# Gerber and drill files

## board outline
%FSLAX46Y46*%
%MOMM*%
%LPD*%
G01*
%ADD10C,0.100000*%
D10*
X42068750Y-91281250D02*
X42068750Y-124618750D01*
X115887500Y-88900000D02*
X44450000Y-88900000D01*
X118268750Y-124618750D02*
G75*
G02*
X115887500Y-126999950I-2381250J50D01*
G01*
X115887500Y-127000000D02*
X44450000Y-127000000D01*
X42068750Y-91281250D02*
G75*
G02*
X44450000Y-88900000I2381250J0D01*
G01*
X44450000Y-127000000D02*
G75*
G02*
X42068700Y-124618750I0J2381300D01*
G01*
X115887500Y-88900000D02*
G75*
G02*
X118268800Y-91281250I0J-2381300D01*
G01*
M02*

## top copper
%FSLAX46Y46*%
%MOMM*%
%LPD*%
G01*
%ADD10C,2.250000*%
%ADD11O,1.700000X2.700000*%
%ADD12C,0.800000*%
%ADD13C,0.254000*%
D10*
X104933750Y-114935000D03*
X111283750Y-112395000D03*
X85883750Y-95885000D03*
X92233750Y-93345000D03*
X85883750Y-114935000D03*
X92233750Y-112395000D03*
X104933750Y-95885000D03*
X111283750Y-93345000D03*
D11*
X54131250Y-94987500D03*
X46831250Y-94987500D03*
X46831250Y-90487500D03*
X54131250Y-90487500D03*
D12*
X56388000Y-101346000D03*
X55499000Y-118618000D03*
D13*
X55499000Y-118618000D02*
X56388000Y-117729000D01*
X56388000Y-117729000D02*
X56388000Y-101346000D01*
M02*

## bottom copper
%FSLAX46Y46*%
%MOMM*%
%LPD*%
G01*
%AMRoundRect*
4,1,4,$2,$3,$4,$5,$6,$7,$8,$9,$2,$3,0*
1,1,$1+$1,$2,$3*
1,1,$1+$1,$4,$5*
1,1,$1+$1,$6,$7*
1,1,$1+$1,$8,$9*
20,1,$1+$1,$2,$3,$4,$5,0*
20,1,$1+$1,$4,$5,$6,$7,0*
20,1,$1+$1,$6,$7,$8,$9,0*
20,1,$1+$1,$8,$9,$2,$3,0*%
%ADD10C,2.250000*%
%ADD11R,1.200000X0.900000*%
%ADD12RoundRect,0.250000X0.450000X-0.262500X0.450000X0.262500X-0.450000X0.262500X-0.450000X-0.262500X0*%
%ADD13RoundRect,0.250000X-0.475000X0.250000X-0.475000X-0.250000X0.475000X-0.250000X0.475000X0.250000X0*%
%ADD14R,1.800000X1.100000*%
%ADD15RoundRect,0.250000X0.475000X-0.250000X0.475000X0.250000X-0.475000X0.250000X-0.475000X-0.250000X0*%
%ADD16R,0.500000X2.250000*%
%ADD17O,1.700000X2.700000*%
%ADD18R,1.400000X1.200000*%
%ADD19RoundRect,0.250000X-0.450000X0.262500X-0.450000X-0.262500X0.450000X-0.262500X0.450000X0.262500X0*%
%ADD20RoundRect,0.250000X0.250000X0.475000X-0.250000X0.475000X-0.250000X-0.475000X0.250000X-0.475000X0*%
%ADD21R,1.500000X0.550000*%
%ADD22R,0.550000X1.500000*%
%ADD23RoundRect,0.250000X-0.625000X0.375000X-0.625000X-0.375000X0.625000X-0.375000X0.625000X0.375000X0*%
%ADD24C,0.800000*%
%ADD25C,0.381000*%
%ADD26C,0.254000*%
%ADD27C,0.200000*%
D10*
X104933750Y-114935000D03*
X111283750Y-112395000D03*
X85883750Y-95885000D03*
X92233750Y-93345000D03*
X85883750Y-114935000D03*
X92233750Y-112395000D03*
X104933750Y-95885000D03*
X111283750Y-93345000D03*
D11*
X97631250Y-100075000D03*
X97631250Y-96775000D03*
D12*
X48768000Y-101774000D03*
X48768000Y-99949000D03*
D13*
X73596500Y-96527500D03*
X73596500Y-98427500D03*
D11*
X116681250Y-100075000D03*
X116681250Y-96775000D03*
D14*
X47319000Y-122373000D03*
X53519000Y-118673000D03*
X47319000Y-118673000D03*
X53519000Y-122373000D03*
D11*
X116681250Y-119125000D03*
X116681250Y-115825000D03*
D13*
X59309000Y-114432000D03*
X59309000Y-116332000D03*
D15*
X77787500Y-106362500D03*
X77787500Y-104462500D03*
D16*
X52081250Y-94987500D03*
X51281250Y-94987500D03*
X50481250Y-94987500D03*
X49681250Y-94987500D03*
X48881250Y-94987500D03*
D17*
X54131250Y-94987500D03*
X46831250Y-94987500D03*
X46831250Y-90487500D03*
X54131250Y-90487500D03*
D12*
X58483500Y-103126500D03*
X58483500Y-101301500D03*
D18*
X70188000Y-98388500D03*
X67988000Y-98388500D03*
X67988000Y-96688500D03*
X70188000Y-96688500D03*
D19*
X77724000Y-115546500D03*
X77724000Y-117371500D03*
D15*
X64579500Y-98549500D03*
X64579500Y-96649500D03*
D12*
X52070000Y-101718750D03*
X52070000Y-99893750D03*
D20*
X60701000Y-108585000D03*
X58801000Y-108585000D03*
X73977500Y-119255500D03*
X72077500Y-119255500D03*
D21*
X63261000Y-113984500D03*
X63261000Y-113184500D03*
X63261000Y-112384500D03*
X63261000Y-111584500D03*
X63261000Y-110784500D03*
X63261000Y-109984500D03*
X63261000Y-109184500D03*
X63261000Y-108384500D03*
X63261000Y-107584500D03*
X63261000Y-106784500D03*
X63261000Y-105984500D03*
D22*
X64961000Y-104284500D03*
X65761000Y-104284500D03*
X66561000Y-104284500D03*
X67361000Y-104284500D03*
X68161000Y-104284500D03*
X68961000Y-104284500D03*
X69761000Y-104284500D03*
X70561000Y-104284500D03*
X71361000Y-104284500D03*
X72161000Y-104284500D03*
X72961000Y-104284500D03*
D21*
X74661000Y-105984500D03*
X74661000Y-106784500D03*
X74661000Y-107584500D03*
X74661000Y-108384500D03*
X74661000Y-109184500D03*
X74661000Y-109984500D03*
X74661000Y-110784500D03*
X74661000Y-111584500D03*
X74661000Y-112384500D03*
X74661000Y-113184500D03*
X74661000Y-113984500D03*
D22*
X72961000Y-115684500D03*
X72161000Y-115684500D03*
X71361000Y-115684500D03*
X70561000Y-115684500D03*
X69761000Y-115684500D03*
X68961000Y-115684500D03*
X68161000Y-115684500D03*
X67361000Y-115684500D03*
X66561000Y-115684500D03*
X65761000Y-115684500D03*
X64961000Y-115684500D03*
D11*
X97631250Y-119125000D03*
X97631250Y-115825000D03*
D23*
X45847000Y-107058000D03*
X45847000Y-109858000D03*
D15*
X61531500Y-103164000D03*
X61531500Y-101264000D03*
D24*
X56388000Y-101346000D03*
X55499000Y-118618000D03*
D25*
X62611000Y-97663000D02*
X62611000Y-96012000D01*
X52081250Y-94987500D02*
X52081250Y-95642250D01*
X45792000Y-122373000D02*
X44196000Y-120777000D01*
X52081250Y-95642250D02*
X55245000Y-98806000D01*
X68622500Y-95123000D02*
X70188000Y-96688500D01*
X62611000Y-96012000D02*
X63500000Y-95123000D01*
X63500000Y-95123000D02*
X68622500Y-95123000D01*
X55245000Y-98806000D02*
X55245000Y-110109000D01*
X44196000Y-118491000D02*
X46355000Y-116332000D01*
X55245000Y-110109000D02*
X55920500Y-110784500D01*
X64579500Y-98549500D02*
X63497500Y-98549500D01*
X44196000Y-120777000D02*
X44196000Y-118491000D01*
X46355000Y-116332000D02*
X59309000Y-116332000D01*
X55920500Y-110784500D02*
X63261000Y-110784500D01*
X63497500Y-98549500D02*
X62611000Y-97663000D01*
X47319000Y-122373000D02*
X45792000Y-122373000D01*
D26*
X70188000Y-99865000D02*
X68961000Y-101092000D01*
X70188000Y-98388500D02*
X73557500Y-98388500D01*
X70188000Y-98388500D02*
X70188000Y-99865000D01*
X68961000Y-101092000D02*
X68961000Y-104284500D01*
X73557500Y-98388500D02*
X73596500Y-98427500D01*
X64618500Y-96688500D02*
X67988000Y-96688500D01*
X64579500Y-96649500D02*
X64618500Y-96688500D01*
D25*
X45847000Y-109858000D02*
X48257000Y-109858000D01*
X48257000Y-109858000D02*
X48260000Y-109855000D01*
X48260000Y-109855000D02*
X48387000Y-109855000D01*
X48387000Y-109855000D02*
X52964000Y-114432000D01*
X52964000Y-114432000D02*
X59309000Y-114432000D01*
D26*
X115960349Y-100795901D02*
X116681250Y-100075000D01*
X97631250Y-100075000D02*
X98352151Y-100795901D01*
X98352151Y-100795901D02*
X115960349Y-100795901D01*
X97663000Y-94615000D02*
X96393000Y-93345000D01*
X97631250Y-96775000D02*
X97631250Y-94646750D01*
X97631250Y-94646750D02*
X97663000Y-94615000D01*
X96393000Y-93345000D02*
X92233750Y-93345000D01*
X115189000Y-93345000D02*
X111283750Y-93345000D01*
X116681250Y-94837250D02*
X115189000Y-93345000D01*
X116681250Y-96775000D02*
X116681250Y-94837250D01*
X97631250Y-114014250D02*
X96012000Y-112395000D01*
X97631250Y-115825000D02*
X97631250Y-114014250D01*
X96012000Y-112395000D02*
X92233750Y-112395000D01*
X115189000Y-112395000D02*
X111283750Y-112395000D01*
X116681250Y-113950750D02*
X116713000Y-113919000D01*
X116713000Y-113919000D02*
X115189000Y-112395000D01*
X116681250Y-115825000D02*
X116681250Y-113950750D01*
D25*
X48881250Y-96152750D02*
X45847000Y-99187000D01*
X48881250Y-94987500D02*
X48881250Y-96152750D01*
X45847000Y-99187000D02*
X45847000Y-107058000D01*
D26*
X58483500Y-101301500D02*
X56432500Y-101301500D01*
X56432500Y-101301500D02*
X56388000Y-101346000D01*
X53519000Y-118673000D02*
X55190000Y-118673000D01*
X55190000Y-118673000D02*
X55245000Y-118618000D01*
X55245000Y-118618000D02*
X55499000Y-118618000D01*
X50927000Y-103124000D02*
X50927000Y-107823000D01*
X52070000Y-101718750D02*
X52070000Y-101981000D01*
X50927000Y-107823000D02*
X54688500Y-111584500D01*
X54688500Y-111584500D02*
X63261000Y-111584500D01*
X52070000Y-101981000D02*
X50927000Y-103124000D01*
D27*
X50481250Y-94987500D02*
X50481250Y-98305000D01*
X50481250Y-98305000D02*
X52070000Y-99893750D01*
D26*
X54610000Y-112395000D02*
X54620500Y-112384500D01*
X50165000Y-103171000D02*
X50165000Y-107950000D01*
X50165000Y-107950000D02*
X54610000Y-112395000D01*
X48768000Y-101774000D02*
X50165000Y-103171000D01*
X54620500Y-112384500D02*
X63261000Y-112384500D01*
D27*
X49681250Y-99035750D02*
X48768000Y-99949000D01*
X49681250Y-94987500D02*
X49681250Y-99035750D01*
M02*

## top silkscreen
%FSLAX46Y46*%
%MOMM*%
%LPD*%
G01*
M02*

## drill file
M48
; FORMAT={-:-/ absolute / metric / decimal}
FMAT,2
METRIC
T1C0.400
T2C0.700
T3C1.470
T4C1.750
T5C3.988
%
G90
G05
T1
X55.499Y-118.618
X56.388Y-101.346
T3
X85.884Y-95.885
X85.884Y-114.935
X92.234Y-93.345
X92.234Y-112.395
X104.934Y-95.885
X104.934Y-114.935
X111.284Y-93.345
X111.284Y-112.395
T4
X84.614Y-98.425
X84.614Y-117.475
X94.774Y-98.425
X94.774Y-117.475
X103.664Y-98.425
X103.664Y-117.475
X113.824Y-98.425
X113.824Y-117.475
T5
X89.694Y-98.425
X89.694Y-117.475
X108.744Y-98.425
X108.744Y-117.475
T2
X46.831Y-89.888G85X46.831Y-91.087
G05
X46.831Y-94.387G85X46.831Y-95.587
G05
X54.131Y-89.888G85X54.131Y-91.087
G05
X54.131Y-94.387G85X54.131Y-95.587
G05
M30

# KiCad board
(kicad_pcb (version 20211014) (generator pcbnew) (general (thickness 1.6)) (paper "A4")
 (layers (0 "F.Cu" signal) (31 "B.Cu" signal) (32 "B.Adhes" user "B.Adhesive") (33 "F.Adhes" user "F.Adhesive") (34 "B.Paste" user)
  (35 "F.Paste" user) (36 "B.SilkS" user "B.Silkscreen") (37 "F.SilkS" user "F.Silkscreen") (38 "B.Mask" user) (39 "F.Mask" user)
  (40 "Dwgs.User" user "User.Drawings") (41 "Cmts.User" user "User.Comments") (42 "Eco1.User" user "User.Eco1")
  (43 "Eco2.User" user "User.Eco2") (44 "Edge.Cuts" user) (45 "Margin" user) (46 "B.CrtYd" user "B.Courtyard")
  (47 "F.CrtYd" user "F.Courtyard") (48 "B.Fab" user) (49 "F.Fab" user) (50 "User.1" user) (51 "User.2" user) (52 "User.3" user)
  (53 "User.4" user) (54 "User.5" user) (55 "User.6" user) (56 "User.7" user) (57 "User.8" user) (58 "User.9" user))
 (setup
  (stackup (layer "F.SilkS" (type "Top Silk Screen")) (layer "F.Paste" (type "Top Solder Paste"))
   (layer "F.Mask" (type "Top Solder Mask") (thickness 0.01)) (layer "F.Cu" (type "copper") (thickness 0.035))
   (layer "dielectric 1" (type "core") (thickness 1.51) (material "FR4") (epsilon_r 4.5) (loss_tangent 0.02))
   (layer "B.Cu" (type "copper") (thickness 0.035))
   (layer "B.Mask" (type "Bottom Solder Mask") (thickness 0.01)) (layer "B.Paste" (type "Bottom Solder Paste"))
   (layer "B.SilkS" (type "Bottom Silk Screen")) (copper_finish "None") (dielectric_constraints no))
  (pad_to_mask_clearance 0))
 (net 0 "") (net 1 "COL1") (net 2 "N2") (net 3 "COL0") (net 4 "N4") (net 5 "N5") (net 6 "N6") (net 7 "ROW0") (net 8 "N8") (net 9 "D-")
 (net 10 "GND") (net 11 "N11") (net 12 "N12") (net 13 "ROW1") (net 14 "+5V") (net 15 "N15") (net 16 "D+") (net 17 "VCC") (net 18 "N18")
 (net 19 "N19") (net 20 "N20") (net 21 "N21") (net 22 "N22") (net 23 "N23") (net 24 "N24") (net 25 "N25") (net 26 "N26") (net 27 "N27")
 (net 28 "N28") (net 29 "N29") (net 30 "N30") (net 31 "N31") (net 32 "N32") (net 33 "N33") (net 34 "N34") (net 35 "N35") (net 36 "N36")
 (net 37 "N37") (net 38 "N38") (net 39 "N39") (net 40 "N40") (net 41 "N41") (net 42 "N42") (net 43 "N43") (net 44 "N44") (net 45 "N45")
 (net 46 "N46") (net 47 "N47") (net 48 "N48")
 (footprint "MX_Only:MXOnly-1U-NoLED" (layer "F.Cu") (at 108.74375 117.475)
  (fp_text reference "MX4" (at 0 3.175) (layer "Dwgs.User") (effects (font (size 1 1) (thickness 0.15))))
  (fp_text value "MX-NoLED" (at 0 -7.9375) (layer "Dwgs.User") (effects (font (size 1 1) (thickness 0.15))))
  (pad "" np_thru_hole circle locked (at 5.08 0 48.0996) (size 1.75 1.75) (drill 1.75) (layers *.Cu *.Mask))
  (pad "" np_thru_hole circle locked (at 0 0) (size 3.9878 3.9878) (drill 3.9878) (layers *.Cu *.Mask))
  (pad "" np_thru_hole circle locked (at -5.08 0 48.0996) (size 1.75 1.75) (drill 1.75) (layers *.Cu *.Mask))
  (pad "1" thru_hole circle locked (at -3.81 -2.54) (size 2.25 2.25) (drill 1.47) (layers *.Cu "B.Mask") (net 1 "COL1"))
  (pad "2" thru_hole circle locked (at 2.54 -5.08) (size 2.25 2.25) (drill 1.47) (layers *.Cu "B.Mask") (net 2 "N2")))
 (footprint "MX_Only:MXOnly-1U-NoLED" (layer "F.Cu") (at 89.69375 98.425)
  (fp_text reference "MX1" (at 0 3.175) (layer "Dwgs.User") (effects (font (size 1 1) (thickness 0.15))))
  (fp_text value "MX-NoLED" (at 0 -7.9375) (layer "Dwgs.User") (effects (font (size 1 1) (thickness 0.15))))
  (pad "" np_thru_hole circle locked (at -5.08 0 48.0996) (size 1.75 1.75) (drill 1.75) (layers *.Cu *.Mask))
  (pad "" np_thru_hole circle locked (at 5.08 0 48.0996) (size 1.75 1.75) (drill 1.75) (layers *.Cu *.Mask))
  (pad "" np_thru_hole circle locked (at 0 0) (size 3.9878 3.9878) (drill 3.9878) (layers *.Cu *.Mask))
  (pad "1" thru_hole circle locked (at -3.81 -2.54) (size 2.25 2.25) (drill 1.47) (layers *.Cu "B.Mask") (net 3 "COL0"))
  (pad "2" thru_hole circle locked (at 2.54 -5.08) (size 2.25 2.25) (drill 1.47) (layers *.Cu "B.Mask") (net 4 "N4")))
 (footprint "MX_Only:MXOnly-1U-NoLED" (layer "F.Cu") (at 89.69375 117.475)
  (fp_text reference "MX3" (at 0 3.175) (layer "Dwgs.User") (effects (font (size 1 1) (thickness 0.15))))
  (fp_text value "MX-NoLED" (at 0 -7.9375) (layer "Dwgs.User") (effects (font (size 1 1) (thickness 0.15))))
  (pad "" np_thru_hole circle locked (at -5.08 0 48.0996) (size 1.75 1.75) (drill 1.75) (layers *.Cu *.Mask))
  (pad "" np_thru_hole circle locked (at 5.08 0 48.0996) (size 1.75 1.75) (drill 1.75) (layers *.Cu *.Mask))
  (pad "" np_thru_hole circle locked (at 0 0) (size 3.9878 3.9878) (drill 3.9878) (layers *.Cu *.Mask))
  (pad "1" thru_hole circle locked (at -3.81 -2.54) (size 2.25 2.25) (drill 1.47) (layers *.Cu "B.Mask") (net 3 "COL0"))
  (pad "2" thru_hole circle locked (at 2.54 -5.08) (size 2.25 2.25) (drill 1.47) (layers *.Cu "B.Mask") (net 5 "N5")))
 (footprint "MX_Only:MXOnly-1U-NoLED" (layer "F.Cu") (at 108.74375 98.425)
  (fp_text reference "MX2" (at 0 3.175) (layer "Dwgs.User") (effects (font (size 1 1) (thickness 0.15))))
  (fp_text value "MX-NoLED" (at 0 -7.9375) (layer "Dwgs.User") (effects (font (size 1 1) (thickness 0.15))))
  (pad "" np_thru_hole circle locked (at -5.08 0 48.0996) (size 1.75 1.75) (drill 1.75) (layers *.Cu *.Mask))
  (pad "" np_thru_hole circle locked (at 0 0) (size 3.9878 3.9878) (drill 3.9878) (layers *.Cu *.Mask))
  (pad "" np_thru_hole circle locked (at 5.08 0 48.0996) (size 1.75 1.75) (drill 1.75) (layers *.Cu *.Mask))
  (pad "1" thru_hole circle locked (at -3.81 -2.54) (size 2.25 2.25) (drill 1.47) (layers *.Cu "B.Mask") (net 1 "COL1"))
  (pad "2" thru_hole circle locked (at 2.54 -5.08) (size 2.25 2.25) (drill 1.47) (layers *.Cu "B.Mask") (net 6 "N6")))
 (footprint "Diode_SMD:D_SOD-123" (layer "B.Cu") (at 97.63125 98.425 90)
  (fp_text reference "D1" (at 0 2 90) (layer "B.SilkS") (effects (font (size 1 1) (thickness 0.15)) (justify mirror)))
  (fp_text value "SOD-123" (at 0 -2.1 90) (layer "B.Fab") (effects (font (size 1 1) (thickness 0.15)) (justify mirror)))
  (pad "1" smd rect (at -1.65 0 90) (size 0.9 1.2) (layers "B.Cu" "B.Paste" "B.Mask") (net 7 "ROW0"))
  (pad "2" smd rect (at 1.65 0 90) (size 0.9 1.2) (layers "B.Cu" "B.Paste" "B.Mask") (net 4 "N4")))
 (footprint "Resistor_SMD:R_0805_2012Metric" (layer "B.Cu") (at 48.768 100.8615 90)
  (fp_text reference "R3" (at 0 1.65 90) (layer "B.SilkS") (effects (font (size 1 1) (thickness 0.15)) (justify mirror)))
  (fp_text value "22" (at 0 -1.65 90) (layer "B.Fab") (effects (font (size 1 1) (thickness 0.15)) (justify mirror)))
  (pad "1" smd roundrect (at -0.9125 0 90) (size 1.025 1.4) (layers "B.Cu" "B.Paste" "B.Mask") (roundrect_rratio 0.243902) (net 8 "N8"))
  (pad "2" smd roundrect (at 0.9125 0 90) (size 1.025 1.4) (layers "B.Cu" "B.Paste" "B.Mask") (roundrect_rratio 0.243902) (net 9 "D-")))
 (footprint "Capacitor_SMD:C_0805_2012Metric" (layer "B.Cu") (at 73.5965 97.4775 -90)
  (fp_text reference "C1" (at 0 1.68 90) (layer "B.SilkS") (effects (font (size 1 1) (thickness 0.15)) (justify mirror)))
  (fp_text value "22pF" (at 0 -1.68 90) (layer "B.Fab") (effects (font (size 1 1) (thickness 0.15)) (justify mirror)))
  (pad "1" smd roundrect (at -0.95 0 270) (size 1 1.45) (layers "B.Cu" "B.Paste" "B.Mask") (roundrect_rratio 0.25) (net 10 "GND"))
  (pad "2" smd roundrect (at 0.95 0 270) (size 1 1.45) (layers "B.Cu" "B.Paste" "B.Mask") (roundrect_rratio 0.25) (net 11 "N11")))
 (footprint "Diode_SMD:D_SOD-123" (layer "B.Cu") (at 116.68125 98.425 90)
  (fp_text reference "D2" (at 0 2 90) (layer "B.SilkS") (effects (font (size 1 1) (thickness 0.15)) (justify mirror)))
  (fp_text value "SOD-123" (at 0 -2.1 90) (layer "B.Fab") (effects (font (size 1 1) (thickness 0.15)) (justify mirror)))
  (pad "1" smd rect (at -1.65 0 90) (size 0.9 1.2) (layers "B.Cu" "B.Paste" "B.Mask") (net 7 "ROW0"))
  (pad "2" smd rect (at 1.65 0 90) (size 0.9 1.2) (layers "B.Cu" "B.Paste" "B.Mask") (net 6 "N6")))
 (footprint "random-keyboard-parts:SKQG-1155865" (layer "B.Cu") (at 50.419 120.523 180)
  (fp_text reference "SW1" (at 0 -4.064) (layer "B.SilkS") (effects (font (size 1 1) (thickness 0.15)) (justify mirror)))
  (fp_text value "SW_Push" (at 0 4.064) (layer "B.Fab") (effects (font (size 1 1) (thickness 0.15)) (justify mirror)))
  (pad "1" smd rect locked (at 3.1 -1.85 180) (size 1.8 1.1) (layers "B.Cu" "B.Paste" "B.Mask") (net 10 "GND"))
  (pad "2" smd rect locked (at -3.1 1.85 180) (size 1.8 1.1) (layers "B.Cu" "B.Paste" "B.Mask") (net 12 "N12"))
  (pad "3" smd rect locked (at 3.1 1.85 180) (size 1.8 1.1) (layers "B.Cu" "B.Paste" "B.Mask"))
  (pad "4" smd rect locked (at -3.1 -1.85 180) (size 1.8 1.1) (layers "B.Cu" "B.Paste" "B.Mask")))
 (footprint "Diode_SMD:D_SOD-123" (layer "B.Cu") (at 116.68125 117.475 90)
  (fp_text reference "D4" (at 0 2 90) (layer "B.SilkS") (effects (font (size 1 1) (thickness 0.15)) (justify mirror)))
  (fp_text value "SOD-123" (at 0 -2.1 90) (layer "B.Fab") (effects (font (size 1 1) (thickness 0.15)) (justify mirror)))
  (pad "1" smd rect (at -1.65 0 90) (size 0.9 1.2) (layers "B.Cu" "B.Paste" "B.Mask") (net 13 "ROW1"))
  (pad "2" smd rect (at 1.65 0 90) (size 0.9 1.2) (layers "B.Cu" "B.Paste" "B.Mask") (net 2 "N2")))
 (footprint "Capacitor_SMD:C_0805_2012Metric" (layer "B.Cu") (at 59.309 115.382 -90)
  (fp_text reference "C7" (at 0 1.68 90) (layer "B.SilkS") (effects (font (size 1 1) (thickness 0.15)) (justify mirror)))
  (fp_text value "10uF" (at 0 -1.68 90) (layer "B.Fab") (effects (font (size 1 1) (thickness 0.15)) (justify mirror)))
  (pad "1" smd roundrect (at -0.95 0 270) (size 1 1.45) (layers "B.Cu" "B.Paste" "B.Mask") (roundrect_rratio 0.25) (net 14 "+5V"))
  (pad "2" smd roundrect (at 0.95 0 270) (size 1 1.45) (layers "B.Cu" "B.Paste" "B.Mask") (roundrect_rratio 0.25) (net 10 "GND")))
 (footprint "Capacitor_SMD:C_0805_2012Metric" (layer "B.Cu") (at 77.7875 105.4125 90)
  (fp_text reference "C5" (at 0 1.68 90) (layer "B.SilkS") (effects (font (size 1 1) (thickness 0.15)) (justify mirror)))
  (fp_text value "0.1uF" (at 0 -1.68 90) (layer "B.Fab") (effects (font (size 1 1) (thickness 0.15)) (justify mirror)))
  (pad "1" smd roundrect (at -0.95 0 90) (size 1 1.45) (layers "B.Cu" "B.Paste" "B.Mask") (roundrect_rratio 0.25) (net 14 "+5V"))
  (pad "2" smd roundrect (at 0.95 0 90) (size 1 1.45) (layers "B.Cu" "B.Paste" "B.Mask") (roundrect_rratio 0.25) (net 10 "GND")))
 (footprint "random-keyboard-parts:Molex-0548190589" (layer "B.Cu") (at 50.48125 90.4875 -90)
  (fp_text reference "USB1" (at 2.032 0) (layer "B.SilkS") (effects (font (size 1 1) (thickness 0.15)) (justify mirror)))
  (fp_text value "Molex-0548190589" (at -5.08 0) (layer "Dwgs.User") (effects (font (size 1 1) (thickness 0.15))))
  (pad "1" smd rect locked (at 4.5 -1.6 270) (size 2.25 0.5) (layers "B.Cu" "B.Paste" "B.Mask") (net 10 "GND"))
  (pad "2" smd rect locked (at 4.5 -0.8 270) (size 2.25 0.5) (layers "B.Cu" "B.Paste" "B.Mask") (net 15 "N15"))
  (pad "3" smd rect locked (at 4.5 0 270) (size 2.25 0.5) (layers "B.Cu" "B.Paste" "B.Mask") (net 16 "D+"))
  (pad "4" smd rect locked (at 4.5 0.8 270) (size 2.25 0.5) (layers "B.Cu" "B.Paste" "B.Mask") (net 9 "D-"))
  (pad "5" smd rect locked (at 4.5 1.6 270) (size 2.25 0.5) (layers "B.Cu" "B.Paste" "B.Mask") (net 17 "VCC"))
  (pad "6" thru_hole oval locked (at 4.5 -3.65 270) (size 2.7 1.7) (drill oval 1.9 0.7) (layers *.Cu *.Mask) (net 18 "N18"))
  (pad "6" thru_hole oval locked (at 4.5 3.65 270) (size 2.7 1.7) (drill oval 1.9 0.7) (layers *.Cu *.Mask) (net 18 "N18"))
  (pad "6" thru_hole oval locked (at 0 3.65 270) (size 2.7 1.7) (drill oval 1.9 0.7) (layers *.Cu *.Mask) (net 18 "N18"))
  (pad "6" thru_hole oval locked (at 0 -3.65 270) (size 2.7 1.7) (drill oval 1.9 0.7) (layers *.Cu *.Mask) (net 18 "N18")))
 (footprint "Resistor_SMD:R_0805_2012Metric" (layer "B.Cu") (at 58.4835 102.214 90)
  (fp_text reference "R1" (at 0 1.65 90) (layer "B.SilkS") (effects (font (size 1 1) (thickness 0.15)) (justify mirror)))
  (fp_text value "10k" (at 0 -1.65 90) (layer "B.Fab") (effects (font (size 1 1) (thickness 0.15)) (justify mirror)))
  (pad "1" smd roundrect (at -0.9125 0 90) (size 1.025 1.4) (layers "B.Cu" "B.Paste" "B.Mask") (roundrect_rratio 0.243902) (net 14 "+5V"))
  (pad "2" smd roundrect (at 0.9125 0 90) (size 1.025 1.4) (layers "B.Cu" "B.Paste" "B.Mask") (roundrect_rratio 0.243902) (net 12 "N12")))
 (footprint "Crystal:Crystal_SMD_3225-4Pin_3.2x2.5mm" (layer "B.Cu") (at 69.088 97.5385 180)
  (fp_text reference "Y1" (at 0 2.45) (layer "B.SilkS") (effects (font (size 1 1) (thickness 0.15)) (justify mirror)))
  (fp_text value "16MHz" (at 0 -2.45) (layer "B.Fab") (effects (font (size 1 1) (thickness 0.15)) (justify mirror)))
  (pad "1" smd rect (at -1.1 -0.85 180) (size 1.4 1.2) (layers "B.Cu" "B.Paste" "B.Mask") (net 11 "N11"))
  (pad "2" smd rect (at 1.1 -0.85 180) (size 1.4 1.2) (layers "B.Cu" "B.Paste" "B.Mask") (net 10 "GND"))
  (pad "3" smd rect (at 1.1 0.85 180) (size 1.4 1.2) (layers "B.Cu" "B.Paste" "B.Mask") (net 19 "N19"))
  (pad "4" smd rect (at -1.1 0.85 180) (size 1.4 1.2) (layers "B.Cu" "B.Paste" "B.Mask") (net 10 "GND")))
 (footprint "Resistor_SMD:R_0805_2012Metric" (layer "B.Cu") (at 77.724 116.459 -90)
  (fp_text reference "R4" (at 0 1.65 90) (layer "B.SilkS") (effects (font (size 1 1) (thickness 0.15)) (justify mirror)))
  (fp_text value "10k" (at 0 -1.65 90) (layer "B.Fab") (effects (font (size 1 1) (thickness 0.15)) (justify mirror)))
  (pad "1" smd roundrect (at -0.9125 0 270) (size 1.025 1.4) (layers "B.Cu" "B.Paste" "B.Mask") (roundrect_rratio 0.243902) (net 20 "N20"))
  (pad "2" smd roundrect (at 0.9125 0 270) (size 1.025 1.4) (layers "B.Cu" "B.Paste" "B.Mask") (roundrect_rratio 0.243902) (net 10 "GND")))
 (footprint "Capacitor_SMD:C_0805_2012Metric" (layer "B.Cu") (at 64.5795 97.5995 90)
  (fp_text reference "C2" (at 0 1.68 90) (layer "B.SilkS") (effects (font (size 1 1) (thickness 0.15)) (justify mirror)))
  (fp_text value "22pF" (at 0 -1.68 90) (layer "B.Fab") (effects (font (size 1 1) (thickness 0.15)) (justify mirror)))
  (pad "1" smd roundrect (at -0.95 0 90) (size 1 1.45) (layers "B.Cu" "B.Paste" "B.Mask") (roundrect_rratio 0.25) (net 10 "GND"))
  (pad "2" smd roundrect (at 0.95 0 90) (size 1 1.45) (layers "B.Cu" "B.Paste" "B.Mask") (roundrect_rratio 0.25) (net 19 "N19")))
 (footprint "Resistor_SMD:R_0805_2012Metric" (layer "B.Cu") (at 52.07 100.80625 90)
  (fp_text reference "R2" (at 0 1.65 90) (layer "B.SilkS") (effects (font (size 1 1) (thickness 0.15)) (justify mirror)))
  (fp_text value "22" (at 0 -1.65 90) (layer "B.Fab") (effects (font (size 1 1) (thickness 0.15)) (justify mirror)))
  (pad "1" smd roundrect (at -0.9125 0 90) (size 1.025 1.4) (layers "B.Cu" "B.Paste" "B.Mask") (roundrect_rratio 0.243902) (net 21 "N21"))
  (pad "2" smd roundrect (at 0.9125 0 90) (size 1.025 1.4) (layers "B.Cu" "B.Paste" "B.Mask") (roundrect_rratio 0.243902) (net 16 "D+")))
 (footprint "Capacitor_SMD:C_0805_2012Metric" (layer "B.Cu") (at 59.751 108.585 180)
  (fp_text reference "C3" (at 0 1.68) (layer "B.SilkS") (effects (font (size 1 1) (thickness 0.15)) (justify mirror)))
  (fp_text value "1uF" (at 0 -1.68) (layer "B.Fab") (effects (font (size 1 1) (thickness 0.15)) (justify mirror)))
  (pad "1" smd roundrect (at -0.95 0 180) (size 1 1.45) (layers "B.Cu" "B.Paste" "B.Mask") (roundrect_rratio 0.25) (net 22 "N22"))
  (pad "2" smd roundrect (at 0.95 0 180) (size 1 1.45) (layers "B.Cu" "B.Paste" "B.Mask") (roundrect_rratio 0.25) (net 10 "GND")))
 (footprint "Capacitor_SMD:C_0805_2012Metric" (layer "B.Cu") (at 73.0275 119.2555 180)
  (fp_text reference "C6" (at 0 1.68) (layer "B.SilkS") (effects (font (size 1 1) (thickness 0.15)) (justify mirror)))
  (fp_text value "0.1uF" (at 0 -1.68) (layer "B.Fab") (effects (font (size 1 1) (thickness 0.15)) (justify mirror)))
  (pad "1" smd roundrect (at -0.95 0 180) (size 1 1.45) (layers "B.Cu" "B.Paste" "B.Mask") (roundrect_rratio 0.25) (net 14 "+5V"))
  (pad "2" smd roundrect (at 0.95 0 180) (size 1 1.45) (layers "B.Cu" "B.Paste" "B.Mask") (roundrect_rratio 0.25) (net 10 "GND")))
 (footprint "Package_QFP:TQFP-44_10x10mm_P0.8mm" (layer "B.Cu") (at 68.961 109.9845)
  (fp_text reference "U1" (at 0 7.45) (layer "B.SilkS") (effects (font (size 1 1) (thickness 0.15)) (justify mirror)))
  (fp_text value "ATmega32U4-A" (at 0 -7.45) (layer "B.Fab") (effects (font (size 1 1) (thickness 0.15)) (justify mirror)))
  (pad "1" smd rect (at -5.7 4) (size 1.5 0.55) (layers "B.Cu" "B.Paste" "B.Mask") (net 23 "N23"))
  (pad "2" smd rect (at -5.7 3.2) (size 1.5 0.55) (layers "B.Cu" "B.Paste" "B.Mask") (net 14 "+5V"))
  (pad "3" smd rect (at -5.7 2.4) (size 1.5 0.55) (layers "B.Cu" "B.Paste" "B.Mask") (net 8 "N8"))
  (pad "4" smd rect (at -5.7 1.6) (size 1.5 0.55) (layers "B.Cu" "B.Paste" "B.Mask") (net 21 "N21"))
  (pad "5" smd rect (at -5.7 0.8) (size 1.5 0.55) (layers "B.Cu" "B.Paste" "B.Mask") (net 10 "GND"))
  (pad "6" smd rect (at -5.7 0) (size 1.5 0.55) (layers "B.Cu" "B.Paste" "B.Mask") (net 22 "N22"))
  (pad "7" smd rect (at -5.7 -0.8) (size 1.5 0.55) (layers "B.Cu" "B.Paste" "B.Mask") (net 14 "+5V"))
  (pad "8" smd rect (at -5.7 -1.6) (size 1.5 0.55) (layers "B.Cu" "B.Paste" "B.Mask") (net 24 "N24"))
  (pad "9" smd rect (at -5.7 -2.4) (size 1.5 0.55) (layers "B.Cu" "B.Paste" "B.Mask") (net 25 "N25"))
  (pad "10" smd rect (at -5.7 -3.2) (size 1.5 0.55) (layers "B.Cu" "B.Paste" "B.Mask") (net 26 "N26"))
  (pad "11" smd rect (at -5.7 -4) (size 1.5 0.55) (layers "B.Cu" "B.Paste" "B.Mask") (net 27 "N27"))
  (pad "12" smd rect (at -4 -5.7 270) (size 1.5 0.55) (layers "B.Cu" "B.Paste" "B.Mask") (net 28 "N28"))
  (pad "13" smd rect (at -3.2 -5.7 270) (size 1.5 0.55) (layers "B.Cu" "B.Paste" "B.Mask") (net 12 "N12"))
  (pad "14" smd rect (at -2.4 -5.7 270) (size 1.5 0.55) (layers "B.Cu" "B.Paste" "B.Mask") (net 14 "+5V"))
  (pad "15" smd rect (at -1.6 -5.7 270) (size 1.5 0.55) (layers "B.Cu" "B.Paste" "B.Mask") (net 10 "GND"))
  (pad "16" smd rect (at -0.8 -5.7 270) (size 1.5 0.55) (layers "B.Cu" "B.Paste" "B.Mask") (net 19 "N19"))
  (pad "17" smd rect (at 0 -5.7 270) (size 1.5 0.55) (layers "B.Cu" "B.Paste" "B.Mask") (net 11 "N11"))
  (pad "18" smd rect (at 0.8 -5.7 270) (size 1.5 0.55) (layers "B.Cu" "B.Paste" "B.Mask") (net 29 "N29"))
  (pad "19" smd rect (at 1.6 -5.7 270) (size 1.5 0.55) (layers "B.Cu" "B.Paste" "B.Mask") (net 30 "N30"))
  (pad "20" smd rect (at 2.4 -5.7 270) (size 1.5 0.55) (layers "B.Cu" "B.Paste" "B.Mask") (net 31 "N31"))
  (pad "21" smd rect (at 3.2 -5.7 270) (size 1.5 0.55) (layers "B.Cu" "B.Paste" "B.Mask") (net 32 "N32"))
  (pad "22" smd rect (at 4 -5.7 270) (size 1.5 0.55) (layers "B.Cu" "B.Paste" "B.Mask") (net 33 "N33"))
  (pad "23" smd rect (at 5.7 -4) (size 1.5 0.55) (layers "B.Cu" "B.Paste" "B.Mask") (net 10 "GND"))
  (pad "24" smd rect (at 5.7 -3.2) (size 1.5 0.55) (layers "B.Cu" "B.Paste" "B.Mask") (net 14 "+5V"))
  (pad "25" smd rect (at 5.7 -2.4) (size 1.5 0.55) (layers "B.Cu" "B.Paste" "B.Mask") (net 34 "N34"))
  (pad "26" smd rect (at 5.7 -1.6) (size 1.5 0.55) (layers "B.Cu" "B.Paste" "B.Mask") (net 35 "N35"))
  (pad "27" smd rect (at 5.7 -0.8) (size 1.5 0.55) (layers "B.Cu" "B.Paste" "B.Mask") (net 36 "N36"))
  (pad "28" smd rect (at 5.7 0) (size 1.5 0.55) (layers "B.Cu" "B.Paste" "B.Mask") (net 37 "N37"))
  (pad "29" smd rect (at 5.7 0.8) (size 1.5 0.55) (layers "B.Cu" "B.Paste" "B.Mask") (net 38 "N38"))
  (pad "30" smd rect (at 5.7 1.6) (size 1.5 0.55) (layers "B.Cu" "B.Paste" "B.Mask") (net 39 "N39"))
  (pad "31" smd rect (at 5.7 2.4) (size 1.5 0.55) (layers "B.Cu" "B.Paste" "B.Mask") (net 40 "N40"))
  (pad "32" smd rect (at 5.7 3.2) (size 1.5 0.55) (layers "B.Cu" "B.Paste" "B.Mask") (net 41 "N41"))
  (pad "33" smd rect (at 5.7 4) (size 1.5 0.55) (layers "B.Cu" "B.Paste" "B.Mask") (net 20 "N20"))
  (pad "34" smd rect (at 4 5.7 270) (size 1.5 0.55) (layers "B.Cu" "B.Paste" "B.Mask") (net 14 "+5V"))
  (pad "35" smd rect (at 3.2 5.7 270) (size 1.5 0.55) (layers "B.Cu" "B.Paste" "B.Mask") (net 10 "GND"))
  (pad "36" smd rect (at 2.4 5.7 270) (size 1.5 0.55) (layers "B.Cu" "B.Paste" "B.Mask") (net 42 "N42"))
  (pad "37" smd rect (at 1.6 5.7 270) (size 1.5 0.55) (layers "B.Cu" "B.Paste" "B.Mask") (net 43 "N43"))
  (pad "38" smd rect (at 0.8 5.7 270) (size 1.5 0.55) (layers "B.Cu" "B.Paste" "B.Mask") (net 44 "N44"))
  (pad "39" smd rect (at 0 5.7 270) (size 1.5 0.55) (layers "B.Cu" "B.Paste" "B.Mask") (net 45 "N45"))
  (pad "40" smd rect (at -0.8 5.7 270) (size 1.5 0.55) (layers "B.Cu" "B.Paste" "B.Mask") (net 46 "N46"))
  (pad "41" smd rect (at -1.6 5.7 270) (size 1.5 0.55) (layers "B.Cu" "B.Paste" "B.Mask") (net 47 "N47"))
  (pad "42" smd rect (at -2.4 5.7 270) (size 1.5 0.55) (layers "B.Cu" "B.Paste" "B.Mask") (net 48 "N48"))
  (pad "43" smd rect (at -3.2 5.7 270) (size 1.5 0.55) (layers "B.Cu" "B.Paste" "B.Mask") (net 10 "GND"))
  (pad "44" smd rect (at -4 5.7 270) (size 1.5 0.55) (layers "B.Cu" "B.Paste" "B.Mask") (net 14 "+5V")))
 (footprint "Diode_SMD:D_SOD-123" (layer "B.Cu") (at 97.63125 117.475 90)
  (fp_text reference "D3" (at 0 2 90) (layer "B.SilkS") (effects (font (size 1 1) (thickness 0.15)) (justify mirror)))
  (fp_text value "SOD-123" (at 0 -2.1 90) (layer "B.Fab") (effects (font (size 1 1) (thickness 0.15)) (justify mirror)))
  (pad "1" smd rect (at -1.65 0 90) (size 0.9 1.2) (layers "B.Cu" "B.Paste" "B.Mask") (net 13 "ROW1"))
  (pad "2" smd rect (at 1.65 0 90) (size 0.9 1.2) (layers "B.Cu" "B.Paste" "B.Mask") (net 5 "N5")))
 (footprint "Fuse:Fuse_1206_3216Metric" (layer "B.Cu") (at 45.847 108.458 -90)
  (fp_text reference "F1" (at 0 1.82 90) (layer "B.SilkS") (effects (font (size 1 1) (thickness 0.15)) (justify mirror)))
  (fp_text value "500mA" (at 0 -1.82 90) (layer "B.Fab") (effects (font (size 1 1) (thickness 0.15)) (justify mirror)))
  (pad "1" smd roundrect (at -1.4 0 270) (size 1.25 1.75) (layers "B.Cu" "B.Paste" "B.Mask") (roundrect_rratio 0.2) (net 17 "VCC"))
  (pad "2" smd roundrect (at 1.4 0 270) (size 1.25 1.75) (layers "B.Cu" "B.Paste" "B.Mask") (roundrect_rratio 0.2) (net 14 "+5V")))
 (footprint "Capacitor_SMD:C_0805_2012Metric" (layer "B.Cu") (at 61.5315 102.214 90)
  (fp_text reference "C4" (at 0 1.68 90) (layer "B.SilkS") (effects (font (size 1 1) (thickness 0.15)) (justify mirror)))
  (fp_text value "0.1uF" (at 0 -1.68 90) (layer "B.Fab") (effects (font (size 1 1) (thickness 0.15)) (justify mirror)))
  (pad "1" smd roundrect (at -0.95 0 90) (size 1 1.45) (layers "B.Cu" "B.Paste" "B.Mask") (roundrect_rratio 0.25) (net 14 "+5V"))
  (pad "2" smd roundrect (at 0.95 0 90) (size 1 1.45) (layers "B.Cu" "B.Paste" "B.Mask") (roundrect_rratio 0.25) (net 10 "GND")))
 (gr_line (start 42.06875 91.28125) (end 42.06875 124.61875) (layer "Edge.Cuts") (width 0.1))
 (gr_line (start 115.8875 88.9) (end 44.45 88.9) (layer "Edge.Cuts") (width 0.1))
 (gr_arc (start 118.26875 124.61875) (mid 117.571298 126.302548) (end 115.8875 127) (layer "Edge.Cuts") (width 0.1))
 (gr_line (start 115.8875 127) (end 44.45 127) (layer "Edge.Cuts") (width 0.1))
 (gr_arc (start 42.06875 91.28125) (mid 42.766202 89.597452) (end 44.45 88.9) (layer "Edge.Cuts") (width 0.1))
 (gr_arc (start 44.45 127) (mid 42.766202 126.302548) (end 42.06875 124.61875) (layer "Edge.Cuts") (width 0.1))
 (gr_arc (start 115.8875 88.9) (mid 117.571298 89.597452) (end 118.26875 91.28125) (layer "Edge.Cuts") (width 0.1))
 (segment (start 62.611 97.663) (end 62.611 96.012) (width 0.381) (layer "B.Cu") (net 10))
 (segment (start 52.08125 94.9875) (end 52.08125 95.64225) (width 0.381) (layer "B.Cu") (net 10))
 (segment (start 45.792 122.373) (end 44.196 120.777) (width 0.381) (layer "B.Cu") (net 10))
 (segment (start 52.08125 95.64225) (end 55.245 98.806) (width 0.381) (layer "B.Cu") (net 10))
 (segment (start 68.6225 95.123) (end 70.188 96.6885) (width 0.381) (layer "B.Cu") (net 10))
 (segment (start 62.611 96.012) (end 63.5 95.123) (width 0.381) (layer "B.Cu") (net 10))
 (segment (start 63.5 95.123) (end 68.6225 95.123) (width 0.381) (layer "B.Cu") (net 10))
 (segment (start 55.245 98.806) (end 55.245 110.109) (width 0.381) (layer "B.Cu") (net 10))
 (segment (start 44.196 118.491) (end 46.355 116.332) (width 0.381) (layer "B.Cu") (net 10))
 (segment (start 55.245 110.109) (end 55.9205 110.7845) (width 0.381) (layer "B.Cu") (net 10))
 (segment (start 64.5795 98.5495) (end 63.4975 98.5495) (width 0.381) (layer "B.Cu") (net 10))
 (segment (start 44.196 120.777) (end 44.196 118.491) (width 0.381) (layer "B.Cu") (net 10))
 (segment (start 46.355 116.332) (end 59.309 116.332) (width 0.381) (layer "B.Cu") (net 10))
 (segment (start 55.9205 110.7845) (end 63.261 110.7845) (width 0.381) (layer "B.Cu") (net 10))
 (segment (start 63.4975 98.5495) (end 62.611 97.663) (width 0.381) (layer "B.Cu") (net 10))
 (segment (start 47.319 122.373) (end 45.792 122.373) (width 0.381) (layer "B.Cu") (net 10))
 (segment (start 70.188 99.865) (end 68.961 101.092) (width 0.254) (layer "B.Cu") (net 11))
 (segment (start 70.188 98.3885) (end 73.5575 98.3885) (width 0.254) (layer "B.Cu") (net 11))
 (segment (start 70.188 98.3885) (end 70.188 99.865) (width 0.254) (layer "B.Cu") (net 11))
 (segment (start 68.961 101.092) (end 68.961 104.2845) (width 0.254) (layer "B.Cu") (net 11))
 (segment (start 73.5575 98.3885) (end 73.5965 98.4275) (width 0.254) (layer "B.Cu") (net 11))
 (segment (start 64.6185 96.6885) (end 67.988 96.6885) (width 0.254) (layer "B.Cu") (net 19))
 (segment (start 64.5795 96.6495) (end 64.6185 96.6885) (width 0.254) (layer "B.Cu") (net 19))
 (segment (start 45.847 109.858) (end 48.257 109.858) (width 0.381) (layer "B.Cu") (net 14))
 (segment (start 48.257 109.858) (end 48.26 109.855) (width 0.381) (layer "B.Cu") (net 14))
 (segment (start 48.26 109.855) (end 48.387 109.855) (width 0.381) (layer "B.Cu") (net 14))
 (segment (start 48.387 109.855) (end 52.964 114.432) (width 0.381) (layer "B.Cu") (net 14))
 (segment (start 52.964 114.432) (end 59.309 114.432) (width 0.381) (layer "B.Cu") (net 14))
 (segment (start 115.960349 100.795901) (end 116.68125 100.075) (width 0.254) (layer "B.Cu") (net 7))
 (segment (start 97.63125 100.075) (end 98.352151 100.795901) (width 0.254) (layer "B.Cu") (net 7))
 (segment (start 98.352151 100.795901) (end 115.960349 100.795901) (width 0.254) (layer "B.Cu") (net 7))
 (segment (start 97.663 94.615) (end 96.393 93.345) (width 0.254) (layer "B.Cu") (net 4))
 (segment (start 97.63125 96.775) (end 97.63125 94.64675) (width 0.254) (layer "B.Cu") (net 4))
 (segment (start 97.63125 94.64675) (end 97.663 94.615) (width 0.254) (layer "B.Cu") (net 4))
 (segment (start 96.393 93.345) (end 92.23375 93.345) (width 0.254) (layer "B.Cu") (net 4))
 (segment (start 115.189 93.345) (end 111.28375 93.345) (width 0.254) (layer "B.Cu") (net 6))
 (segment (start 116.68125 94.83725) (end 115.189 93.345) (width 0.254) (layer "B.Cu") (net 6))
 (segment (start 116.68125 96.775) (end 116.68125 94.83725) (width 0.254) (layer "B.Cu") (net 6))
 (segment (start 97.63125 114.01425) (end 96.012 112.395) (width 0.254) (layer "B.Cu") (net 5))
 (segment (start 97.63125 115.825) (end 97.63125 114.01425) (width 0.254) (layer "B.Cu") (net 5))
 (segment (start 96.012 112.395) (end 92.23375 112.395) (width 0.254) (layer "B.Cu") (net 5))
 (segment (start 115.189 112.395) (end 111.28375 112.395) (width 0.254) (layer "B.Cu") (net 2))
 (segment (start 116.68125 113.95075) (end 116.713 113.919) (width 0.254) (layer "B.Cu") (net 2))
 (segment (start 116.713 113.919) (end 115.189 112.395) (width 0.254) (layer "B.Cu") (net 2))
 (segment (start 116.68125 115.825) (end 116.68125 113.95075) (width 0.254) (layer "B.Cu") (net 2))
 (segment (start 48.88125 96.15275) (end 45.847 99.187) (width 0.381) (layer "B.Cu") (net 17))
 (segment (start 48.88125 94.9875) (end 48.88125 96.15275) (width 0.381) (layer "B.Cu") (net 17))
 (segment (start 45.847 99.187) (end 45.847 107.058) (width 0.381) (layer "B.Cu") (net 17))
 (segment (start 55.499 118.618) (end 56.388 117.729) (width 0.254) (layer "F.Cu") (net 12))
 (segment (start 56.388 117.729) (end 56.388 101.346) (width 0.254) (layer "F.Cu") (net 12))
 (via (at 56.388 101.346) (size 0.8) (drill 0.4) (layers "F.Cu" "B.Cu") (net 12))
 (via (at 55.499 118.618) (size 0.8) (drill 0.4) (layers "F.Cu" "B.Cu") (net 12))
 (segment (start 58.4835 101.3015) (end 56.4325 101.3015) (width 0.254) (layer "B.Cu") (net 12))
 (segment (start 56.4325 101.3015) (end 56.388 101.346) (width 0.254) (layer "B.Cu") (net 12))
 (segment (start 53.519 118.673) (end 55.19 118.673) (width 0.254) (layer "B.Cu") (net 12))
 (segment (start 55.19 118.673) (end 55.245 118.618) (width 0.254) (layer "B.Cu") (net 12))
 (segment (start 55.245 118.618) (end 55.499 118.618) (width 0.254) (layer "B.Cu") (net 12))
 (segment (start 50.927 103.124) (end 50.927 107.823) (width 0.254) (layer "B.Cu") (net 21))
 (segment (start 52.07 101.71875) (end 52.07 101.981) (width 0.254) (layer "B.Cu") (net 21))
 (segment (start 50.927 107.823) (end 54.6885 111.5845) (width 0.254) (layer "B.Cu") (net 21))
 (segment (start 54.6885 111.5845) (end 63.261 111.5845) (width 0.254) (layer "B.Cu") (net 21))
 (segment (start 52.07 101.981) (end 50.927 103.124) (width 0.254) (layer "B.Cu") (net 21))
 (segment (start 50.48125 94.9875) (end 50.48125 98.305) (width 0.2) (layer "B.Cu") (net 16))
 (segment (start 50.48125 98.305) (end 52.07 99.89375) (width 0.2) (layer "B.Cu") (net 16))
 (segment (start 54.61 112.395) (end 54.6205 112.3845) (width 0.254) (layer "B.Cu") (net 8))
 (segment (start 50.165 103.171) (end 50.165 107.95) (width 0.254) (layer "B.Cu") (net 8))
 (segment (start 50.165 107.95) (end 54.61 112.395) (width 0.254) (layer "B.Cu") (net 8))
 (segment (start 48.768 101.774) (end 50.165 103.171) (width 0.254) (layer "B.Cu") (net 8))
 (segment (start 54.6205 112.3845) (end 63.261 112.3845) (width 0.254) (layer "B.Cu") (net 8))
 (segment (start 49.68125 99.03575) (end 48.768 99.949) (width 0.2) (layer "B.Cu") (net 9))
 (segment (start 49.68125 94.9875) (end 49.68125 99.03575) (width 0.2) (layer "B.Cu") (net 9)))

